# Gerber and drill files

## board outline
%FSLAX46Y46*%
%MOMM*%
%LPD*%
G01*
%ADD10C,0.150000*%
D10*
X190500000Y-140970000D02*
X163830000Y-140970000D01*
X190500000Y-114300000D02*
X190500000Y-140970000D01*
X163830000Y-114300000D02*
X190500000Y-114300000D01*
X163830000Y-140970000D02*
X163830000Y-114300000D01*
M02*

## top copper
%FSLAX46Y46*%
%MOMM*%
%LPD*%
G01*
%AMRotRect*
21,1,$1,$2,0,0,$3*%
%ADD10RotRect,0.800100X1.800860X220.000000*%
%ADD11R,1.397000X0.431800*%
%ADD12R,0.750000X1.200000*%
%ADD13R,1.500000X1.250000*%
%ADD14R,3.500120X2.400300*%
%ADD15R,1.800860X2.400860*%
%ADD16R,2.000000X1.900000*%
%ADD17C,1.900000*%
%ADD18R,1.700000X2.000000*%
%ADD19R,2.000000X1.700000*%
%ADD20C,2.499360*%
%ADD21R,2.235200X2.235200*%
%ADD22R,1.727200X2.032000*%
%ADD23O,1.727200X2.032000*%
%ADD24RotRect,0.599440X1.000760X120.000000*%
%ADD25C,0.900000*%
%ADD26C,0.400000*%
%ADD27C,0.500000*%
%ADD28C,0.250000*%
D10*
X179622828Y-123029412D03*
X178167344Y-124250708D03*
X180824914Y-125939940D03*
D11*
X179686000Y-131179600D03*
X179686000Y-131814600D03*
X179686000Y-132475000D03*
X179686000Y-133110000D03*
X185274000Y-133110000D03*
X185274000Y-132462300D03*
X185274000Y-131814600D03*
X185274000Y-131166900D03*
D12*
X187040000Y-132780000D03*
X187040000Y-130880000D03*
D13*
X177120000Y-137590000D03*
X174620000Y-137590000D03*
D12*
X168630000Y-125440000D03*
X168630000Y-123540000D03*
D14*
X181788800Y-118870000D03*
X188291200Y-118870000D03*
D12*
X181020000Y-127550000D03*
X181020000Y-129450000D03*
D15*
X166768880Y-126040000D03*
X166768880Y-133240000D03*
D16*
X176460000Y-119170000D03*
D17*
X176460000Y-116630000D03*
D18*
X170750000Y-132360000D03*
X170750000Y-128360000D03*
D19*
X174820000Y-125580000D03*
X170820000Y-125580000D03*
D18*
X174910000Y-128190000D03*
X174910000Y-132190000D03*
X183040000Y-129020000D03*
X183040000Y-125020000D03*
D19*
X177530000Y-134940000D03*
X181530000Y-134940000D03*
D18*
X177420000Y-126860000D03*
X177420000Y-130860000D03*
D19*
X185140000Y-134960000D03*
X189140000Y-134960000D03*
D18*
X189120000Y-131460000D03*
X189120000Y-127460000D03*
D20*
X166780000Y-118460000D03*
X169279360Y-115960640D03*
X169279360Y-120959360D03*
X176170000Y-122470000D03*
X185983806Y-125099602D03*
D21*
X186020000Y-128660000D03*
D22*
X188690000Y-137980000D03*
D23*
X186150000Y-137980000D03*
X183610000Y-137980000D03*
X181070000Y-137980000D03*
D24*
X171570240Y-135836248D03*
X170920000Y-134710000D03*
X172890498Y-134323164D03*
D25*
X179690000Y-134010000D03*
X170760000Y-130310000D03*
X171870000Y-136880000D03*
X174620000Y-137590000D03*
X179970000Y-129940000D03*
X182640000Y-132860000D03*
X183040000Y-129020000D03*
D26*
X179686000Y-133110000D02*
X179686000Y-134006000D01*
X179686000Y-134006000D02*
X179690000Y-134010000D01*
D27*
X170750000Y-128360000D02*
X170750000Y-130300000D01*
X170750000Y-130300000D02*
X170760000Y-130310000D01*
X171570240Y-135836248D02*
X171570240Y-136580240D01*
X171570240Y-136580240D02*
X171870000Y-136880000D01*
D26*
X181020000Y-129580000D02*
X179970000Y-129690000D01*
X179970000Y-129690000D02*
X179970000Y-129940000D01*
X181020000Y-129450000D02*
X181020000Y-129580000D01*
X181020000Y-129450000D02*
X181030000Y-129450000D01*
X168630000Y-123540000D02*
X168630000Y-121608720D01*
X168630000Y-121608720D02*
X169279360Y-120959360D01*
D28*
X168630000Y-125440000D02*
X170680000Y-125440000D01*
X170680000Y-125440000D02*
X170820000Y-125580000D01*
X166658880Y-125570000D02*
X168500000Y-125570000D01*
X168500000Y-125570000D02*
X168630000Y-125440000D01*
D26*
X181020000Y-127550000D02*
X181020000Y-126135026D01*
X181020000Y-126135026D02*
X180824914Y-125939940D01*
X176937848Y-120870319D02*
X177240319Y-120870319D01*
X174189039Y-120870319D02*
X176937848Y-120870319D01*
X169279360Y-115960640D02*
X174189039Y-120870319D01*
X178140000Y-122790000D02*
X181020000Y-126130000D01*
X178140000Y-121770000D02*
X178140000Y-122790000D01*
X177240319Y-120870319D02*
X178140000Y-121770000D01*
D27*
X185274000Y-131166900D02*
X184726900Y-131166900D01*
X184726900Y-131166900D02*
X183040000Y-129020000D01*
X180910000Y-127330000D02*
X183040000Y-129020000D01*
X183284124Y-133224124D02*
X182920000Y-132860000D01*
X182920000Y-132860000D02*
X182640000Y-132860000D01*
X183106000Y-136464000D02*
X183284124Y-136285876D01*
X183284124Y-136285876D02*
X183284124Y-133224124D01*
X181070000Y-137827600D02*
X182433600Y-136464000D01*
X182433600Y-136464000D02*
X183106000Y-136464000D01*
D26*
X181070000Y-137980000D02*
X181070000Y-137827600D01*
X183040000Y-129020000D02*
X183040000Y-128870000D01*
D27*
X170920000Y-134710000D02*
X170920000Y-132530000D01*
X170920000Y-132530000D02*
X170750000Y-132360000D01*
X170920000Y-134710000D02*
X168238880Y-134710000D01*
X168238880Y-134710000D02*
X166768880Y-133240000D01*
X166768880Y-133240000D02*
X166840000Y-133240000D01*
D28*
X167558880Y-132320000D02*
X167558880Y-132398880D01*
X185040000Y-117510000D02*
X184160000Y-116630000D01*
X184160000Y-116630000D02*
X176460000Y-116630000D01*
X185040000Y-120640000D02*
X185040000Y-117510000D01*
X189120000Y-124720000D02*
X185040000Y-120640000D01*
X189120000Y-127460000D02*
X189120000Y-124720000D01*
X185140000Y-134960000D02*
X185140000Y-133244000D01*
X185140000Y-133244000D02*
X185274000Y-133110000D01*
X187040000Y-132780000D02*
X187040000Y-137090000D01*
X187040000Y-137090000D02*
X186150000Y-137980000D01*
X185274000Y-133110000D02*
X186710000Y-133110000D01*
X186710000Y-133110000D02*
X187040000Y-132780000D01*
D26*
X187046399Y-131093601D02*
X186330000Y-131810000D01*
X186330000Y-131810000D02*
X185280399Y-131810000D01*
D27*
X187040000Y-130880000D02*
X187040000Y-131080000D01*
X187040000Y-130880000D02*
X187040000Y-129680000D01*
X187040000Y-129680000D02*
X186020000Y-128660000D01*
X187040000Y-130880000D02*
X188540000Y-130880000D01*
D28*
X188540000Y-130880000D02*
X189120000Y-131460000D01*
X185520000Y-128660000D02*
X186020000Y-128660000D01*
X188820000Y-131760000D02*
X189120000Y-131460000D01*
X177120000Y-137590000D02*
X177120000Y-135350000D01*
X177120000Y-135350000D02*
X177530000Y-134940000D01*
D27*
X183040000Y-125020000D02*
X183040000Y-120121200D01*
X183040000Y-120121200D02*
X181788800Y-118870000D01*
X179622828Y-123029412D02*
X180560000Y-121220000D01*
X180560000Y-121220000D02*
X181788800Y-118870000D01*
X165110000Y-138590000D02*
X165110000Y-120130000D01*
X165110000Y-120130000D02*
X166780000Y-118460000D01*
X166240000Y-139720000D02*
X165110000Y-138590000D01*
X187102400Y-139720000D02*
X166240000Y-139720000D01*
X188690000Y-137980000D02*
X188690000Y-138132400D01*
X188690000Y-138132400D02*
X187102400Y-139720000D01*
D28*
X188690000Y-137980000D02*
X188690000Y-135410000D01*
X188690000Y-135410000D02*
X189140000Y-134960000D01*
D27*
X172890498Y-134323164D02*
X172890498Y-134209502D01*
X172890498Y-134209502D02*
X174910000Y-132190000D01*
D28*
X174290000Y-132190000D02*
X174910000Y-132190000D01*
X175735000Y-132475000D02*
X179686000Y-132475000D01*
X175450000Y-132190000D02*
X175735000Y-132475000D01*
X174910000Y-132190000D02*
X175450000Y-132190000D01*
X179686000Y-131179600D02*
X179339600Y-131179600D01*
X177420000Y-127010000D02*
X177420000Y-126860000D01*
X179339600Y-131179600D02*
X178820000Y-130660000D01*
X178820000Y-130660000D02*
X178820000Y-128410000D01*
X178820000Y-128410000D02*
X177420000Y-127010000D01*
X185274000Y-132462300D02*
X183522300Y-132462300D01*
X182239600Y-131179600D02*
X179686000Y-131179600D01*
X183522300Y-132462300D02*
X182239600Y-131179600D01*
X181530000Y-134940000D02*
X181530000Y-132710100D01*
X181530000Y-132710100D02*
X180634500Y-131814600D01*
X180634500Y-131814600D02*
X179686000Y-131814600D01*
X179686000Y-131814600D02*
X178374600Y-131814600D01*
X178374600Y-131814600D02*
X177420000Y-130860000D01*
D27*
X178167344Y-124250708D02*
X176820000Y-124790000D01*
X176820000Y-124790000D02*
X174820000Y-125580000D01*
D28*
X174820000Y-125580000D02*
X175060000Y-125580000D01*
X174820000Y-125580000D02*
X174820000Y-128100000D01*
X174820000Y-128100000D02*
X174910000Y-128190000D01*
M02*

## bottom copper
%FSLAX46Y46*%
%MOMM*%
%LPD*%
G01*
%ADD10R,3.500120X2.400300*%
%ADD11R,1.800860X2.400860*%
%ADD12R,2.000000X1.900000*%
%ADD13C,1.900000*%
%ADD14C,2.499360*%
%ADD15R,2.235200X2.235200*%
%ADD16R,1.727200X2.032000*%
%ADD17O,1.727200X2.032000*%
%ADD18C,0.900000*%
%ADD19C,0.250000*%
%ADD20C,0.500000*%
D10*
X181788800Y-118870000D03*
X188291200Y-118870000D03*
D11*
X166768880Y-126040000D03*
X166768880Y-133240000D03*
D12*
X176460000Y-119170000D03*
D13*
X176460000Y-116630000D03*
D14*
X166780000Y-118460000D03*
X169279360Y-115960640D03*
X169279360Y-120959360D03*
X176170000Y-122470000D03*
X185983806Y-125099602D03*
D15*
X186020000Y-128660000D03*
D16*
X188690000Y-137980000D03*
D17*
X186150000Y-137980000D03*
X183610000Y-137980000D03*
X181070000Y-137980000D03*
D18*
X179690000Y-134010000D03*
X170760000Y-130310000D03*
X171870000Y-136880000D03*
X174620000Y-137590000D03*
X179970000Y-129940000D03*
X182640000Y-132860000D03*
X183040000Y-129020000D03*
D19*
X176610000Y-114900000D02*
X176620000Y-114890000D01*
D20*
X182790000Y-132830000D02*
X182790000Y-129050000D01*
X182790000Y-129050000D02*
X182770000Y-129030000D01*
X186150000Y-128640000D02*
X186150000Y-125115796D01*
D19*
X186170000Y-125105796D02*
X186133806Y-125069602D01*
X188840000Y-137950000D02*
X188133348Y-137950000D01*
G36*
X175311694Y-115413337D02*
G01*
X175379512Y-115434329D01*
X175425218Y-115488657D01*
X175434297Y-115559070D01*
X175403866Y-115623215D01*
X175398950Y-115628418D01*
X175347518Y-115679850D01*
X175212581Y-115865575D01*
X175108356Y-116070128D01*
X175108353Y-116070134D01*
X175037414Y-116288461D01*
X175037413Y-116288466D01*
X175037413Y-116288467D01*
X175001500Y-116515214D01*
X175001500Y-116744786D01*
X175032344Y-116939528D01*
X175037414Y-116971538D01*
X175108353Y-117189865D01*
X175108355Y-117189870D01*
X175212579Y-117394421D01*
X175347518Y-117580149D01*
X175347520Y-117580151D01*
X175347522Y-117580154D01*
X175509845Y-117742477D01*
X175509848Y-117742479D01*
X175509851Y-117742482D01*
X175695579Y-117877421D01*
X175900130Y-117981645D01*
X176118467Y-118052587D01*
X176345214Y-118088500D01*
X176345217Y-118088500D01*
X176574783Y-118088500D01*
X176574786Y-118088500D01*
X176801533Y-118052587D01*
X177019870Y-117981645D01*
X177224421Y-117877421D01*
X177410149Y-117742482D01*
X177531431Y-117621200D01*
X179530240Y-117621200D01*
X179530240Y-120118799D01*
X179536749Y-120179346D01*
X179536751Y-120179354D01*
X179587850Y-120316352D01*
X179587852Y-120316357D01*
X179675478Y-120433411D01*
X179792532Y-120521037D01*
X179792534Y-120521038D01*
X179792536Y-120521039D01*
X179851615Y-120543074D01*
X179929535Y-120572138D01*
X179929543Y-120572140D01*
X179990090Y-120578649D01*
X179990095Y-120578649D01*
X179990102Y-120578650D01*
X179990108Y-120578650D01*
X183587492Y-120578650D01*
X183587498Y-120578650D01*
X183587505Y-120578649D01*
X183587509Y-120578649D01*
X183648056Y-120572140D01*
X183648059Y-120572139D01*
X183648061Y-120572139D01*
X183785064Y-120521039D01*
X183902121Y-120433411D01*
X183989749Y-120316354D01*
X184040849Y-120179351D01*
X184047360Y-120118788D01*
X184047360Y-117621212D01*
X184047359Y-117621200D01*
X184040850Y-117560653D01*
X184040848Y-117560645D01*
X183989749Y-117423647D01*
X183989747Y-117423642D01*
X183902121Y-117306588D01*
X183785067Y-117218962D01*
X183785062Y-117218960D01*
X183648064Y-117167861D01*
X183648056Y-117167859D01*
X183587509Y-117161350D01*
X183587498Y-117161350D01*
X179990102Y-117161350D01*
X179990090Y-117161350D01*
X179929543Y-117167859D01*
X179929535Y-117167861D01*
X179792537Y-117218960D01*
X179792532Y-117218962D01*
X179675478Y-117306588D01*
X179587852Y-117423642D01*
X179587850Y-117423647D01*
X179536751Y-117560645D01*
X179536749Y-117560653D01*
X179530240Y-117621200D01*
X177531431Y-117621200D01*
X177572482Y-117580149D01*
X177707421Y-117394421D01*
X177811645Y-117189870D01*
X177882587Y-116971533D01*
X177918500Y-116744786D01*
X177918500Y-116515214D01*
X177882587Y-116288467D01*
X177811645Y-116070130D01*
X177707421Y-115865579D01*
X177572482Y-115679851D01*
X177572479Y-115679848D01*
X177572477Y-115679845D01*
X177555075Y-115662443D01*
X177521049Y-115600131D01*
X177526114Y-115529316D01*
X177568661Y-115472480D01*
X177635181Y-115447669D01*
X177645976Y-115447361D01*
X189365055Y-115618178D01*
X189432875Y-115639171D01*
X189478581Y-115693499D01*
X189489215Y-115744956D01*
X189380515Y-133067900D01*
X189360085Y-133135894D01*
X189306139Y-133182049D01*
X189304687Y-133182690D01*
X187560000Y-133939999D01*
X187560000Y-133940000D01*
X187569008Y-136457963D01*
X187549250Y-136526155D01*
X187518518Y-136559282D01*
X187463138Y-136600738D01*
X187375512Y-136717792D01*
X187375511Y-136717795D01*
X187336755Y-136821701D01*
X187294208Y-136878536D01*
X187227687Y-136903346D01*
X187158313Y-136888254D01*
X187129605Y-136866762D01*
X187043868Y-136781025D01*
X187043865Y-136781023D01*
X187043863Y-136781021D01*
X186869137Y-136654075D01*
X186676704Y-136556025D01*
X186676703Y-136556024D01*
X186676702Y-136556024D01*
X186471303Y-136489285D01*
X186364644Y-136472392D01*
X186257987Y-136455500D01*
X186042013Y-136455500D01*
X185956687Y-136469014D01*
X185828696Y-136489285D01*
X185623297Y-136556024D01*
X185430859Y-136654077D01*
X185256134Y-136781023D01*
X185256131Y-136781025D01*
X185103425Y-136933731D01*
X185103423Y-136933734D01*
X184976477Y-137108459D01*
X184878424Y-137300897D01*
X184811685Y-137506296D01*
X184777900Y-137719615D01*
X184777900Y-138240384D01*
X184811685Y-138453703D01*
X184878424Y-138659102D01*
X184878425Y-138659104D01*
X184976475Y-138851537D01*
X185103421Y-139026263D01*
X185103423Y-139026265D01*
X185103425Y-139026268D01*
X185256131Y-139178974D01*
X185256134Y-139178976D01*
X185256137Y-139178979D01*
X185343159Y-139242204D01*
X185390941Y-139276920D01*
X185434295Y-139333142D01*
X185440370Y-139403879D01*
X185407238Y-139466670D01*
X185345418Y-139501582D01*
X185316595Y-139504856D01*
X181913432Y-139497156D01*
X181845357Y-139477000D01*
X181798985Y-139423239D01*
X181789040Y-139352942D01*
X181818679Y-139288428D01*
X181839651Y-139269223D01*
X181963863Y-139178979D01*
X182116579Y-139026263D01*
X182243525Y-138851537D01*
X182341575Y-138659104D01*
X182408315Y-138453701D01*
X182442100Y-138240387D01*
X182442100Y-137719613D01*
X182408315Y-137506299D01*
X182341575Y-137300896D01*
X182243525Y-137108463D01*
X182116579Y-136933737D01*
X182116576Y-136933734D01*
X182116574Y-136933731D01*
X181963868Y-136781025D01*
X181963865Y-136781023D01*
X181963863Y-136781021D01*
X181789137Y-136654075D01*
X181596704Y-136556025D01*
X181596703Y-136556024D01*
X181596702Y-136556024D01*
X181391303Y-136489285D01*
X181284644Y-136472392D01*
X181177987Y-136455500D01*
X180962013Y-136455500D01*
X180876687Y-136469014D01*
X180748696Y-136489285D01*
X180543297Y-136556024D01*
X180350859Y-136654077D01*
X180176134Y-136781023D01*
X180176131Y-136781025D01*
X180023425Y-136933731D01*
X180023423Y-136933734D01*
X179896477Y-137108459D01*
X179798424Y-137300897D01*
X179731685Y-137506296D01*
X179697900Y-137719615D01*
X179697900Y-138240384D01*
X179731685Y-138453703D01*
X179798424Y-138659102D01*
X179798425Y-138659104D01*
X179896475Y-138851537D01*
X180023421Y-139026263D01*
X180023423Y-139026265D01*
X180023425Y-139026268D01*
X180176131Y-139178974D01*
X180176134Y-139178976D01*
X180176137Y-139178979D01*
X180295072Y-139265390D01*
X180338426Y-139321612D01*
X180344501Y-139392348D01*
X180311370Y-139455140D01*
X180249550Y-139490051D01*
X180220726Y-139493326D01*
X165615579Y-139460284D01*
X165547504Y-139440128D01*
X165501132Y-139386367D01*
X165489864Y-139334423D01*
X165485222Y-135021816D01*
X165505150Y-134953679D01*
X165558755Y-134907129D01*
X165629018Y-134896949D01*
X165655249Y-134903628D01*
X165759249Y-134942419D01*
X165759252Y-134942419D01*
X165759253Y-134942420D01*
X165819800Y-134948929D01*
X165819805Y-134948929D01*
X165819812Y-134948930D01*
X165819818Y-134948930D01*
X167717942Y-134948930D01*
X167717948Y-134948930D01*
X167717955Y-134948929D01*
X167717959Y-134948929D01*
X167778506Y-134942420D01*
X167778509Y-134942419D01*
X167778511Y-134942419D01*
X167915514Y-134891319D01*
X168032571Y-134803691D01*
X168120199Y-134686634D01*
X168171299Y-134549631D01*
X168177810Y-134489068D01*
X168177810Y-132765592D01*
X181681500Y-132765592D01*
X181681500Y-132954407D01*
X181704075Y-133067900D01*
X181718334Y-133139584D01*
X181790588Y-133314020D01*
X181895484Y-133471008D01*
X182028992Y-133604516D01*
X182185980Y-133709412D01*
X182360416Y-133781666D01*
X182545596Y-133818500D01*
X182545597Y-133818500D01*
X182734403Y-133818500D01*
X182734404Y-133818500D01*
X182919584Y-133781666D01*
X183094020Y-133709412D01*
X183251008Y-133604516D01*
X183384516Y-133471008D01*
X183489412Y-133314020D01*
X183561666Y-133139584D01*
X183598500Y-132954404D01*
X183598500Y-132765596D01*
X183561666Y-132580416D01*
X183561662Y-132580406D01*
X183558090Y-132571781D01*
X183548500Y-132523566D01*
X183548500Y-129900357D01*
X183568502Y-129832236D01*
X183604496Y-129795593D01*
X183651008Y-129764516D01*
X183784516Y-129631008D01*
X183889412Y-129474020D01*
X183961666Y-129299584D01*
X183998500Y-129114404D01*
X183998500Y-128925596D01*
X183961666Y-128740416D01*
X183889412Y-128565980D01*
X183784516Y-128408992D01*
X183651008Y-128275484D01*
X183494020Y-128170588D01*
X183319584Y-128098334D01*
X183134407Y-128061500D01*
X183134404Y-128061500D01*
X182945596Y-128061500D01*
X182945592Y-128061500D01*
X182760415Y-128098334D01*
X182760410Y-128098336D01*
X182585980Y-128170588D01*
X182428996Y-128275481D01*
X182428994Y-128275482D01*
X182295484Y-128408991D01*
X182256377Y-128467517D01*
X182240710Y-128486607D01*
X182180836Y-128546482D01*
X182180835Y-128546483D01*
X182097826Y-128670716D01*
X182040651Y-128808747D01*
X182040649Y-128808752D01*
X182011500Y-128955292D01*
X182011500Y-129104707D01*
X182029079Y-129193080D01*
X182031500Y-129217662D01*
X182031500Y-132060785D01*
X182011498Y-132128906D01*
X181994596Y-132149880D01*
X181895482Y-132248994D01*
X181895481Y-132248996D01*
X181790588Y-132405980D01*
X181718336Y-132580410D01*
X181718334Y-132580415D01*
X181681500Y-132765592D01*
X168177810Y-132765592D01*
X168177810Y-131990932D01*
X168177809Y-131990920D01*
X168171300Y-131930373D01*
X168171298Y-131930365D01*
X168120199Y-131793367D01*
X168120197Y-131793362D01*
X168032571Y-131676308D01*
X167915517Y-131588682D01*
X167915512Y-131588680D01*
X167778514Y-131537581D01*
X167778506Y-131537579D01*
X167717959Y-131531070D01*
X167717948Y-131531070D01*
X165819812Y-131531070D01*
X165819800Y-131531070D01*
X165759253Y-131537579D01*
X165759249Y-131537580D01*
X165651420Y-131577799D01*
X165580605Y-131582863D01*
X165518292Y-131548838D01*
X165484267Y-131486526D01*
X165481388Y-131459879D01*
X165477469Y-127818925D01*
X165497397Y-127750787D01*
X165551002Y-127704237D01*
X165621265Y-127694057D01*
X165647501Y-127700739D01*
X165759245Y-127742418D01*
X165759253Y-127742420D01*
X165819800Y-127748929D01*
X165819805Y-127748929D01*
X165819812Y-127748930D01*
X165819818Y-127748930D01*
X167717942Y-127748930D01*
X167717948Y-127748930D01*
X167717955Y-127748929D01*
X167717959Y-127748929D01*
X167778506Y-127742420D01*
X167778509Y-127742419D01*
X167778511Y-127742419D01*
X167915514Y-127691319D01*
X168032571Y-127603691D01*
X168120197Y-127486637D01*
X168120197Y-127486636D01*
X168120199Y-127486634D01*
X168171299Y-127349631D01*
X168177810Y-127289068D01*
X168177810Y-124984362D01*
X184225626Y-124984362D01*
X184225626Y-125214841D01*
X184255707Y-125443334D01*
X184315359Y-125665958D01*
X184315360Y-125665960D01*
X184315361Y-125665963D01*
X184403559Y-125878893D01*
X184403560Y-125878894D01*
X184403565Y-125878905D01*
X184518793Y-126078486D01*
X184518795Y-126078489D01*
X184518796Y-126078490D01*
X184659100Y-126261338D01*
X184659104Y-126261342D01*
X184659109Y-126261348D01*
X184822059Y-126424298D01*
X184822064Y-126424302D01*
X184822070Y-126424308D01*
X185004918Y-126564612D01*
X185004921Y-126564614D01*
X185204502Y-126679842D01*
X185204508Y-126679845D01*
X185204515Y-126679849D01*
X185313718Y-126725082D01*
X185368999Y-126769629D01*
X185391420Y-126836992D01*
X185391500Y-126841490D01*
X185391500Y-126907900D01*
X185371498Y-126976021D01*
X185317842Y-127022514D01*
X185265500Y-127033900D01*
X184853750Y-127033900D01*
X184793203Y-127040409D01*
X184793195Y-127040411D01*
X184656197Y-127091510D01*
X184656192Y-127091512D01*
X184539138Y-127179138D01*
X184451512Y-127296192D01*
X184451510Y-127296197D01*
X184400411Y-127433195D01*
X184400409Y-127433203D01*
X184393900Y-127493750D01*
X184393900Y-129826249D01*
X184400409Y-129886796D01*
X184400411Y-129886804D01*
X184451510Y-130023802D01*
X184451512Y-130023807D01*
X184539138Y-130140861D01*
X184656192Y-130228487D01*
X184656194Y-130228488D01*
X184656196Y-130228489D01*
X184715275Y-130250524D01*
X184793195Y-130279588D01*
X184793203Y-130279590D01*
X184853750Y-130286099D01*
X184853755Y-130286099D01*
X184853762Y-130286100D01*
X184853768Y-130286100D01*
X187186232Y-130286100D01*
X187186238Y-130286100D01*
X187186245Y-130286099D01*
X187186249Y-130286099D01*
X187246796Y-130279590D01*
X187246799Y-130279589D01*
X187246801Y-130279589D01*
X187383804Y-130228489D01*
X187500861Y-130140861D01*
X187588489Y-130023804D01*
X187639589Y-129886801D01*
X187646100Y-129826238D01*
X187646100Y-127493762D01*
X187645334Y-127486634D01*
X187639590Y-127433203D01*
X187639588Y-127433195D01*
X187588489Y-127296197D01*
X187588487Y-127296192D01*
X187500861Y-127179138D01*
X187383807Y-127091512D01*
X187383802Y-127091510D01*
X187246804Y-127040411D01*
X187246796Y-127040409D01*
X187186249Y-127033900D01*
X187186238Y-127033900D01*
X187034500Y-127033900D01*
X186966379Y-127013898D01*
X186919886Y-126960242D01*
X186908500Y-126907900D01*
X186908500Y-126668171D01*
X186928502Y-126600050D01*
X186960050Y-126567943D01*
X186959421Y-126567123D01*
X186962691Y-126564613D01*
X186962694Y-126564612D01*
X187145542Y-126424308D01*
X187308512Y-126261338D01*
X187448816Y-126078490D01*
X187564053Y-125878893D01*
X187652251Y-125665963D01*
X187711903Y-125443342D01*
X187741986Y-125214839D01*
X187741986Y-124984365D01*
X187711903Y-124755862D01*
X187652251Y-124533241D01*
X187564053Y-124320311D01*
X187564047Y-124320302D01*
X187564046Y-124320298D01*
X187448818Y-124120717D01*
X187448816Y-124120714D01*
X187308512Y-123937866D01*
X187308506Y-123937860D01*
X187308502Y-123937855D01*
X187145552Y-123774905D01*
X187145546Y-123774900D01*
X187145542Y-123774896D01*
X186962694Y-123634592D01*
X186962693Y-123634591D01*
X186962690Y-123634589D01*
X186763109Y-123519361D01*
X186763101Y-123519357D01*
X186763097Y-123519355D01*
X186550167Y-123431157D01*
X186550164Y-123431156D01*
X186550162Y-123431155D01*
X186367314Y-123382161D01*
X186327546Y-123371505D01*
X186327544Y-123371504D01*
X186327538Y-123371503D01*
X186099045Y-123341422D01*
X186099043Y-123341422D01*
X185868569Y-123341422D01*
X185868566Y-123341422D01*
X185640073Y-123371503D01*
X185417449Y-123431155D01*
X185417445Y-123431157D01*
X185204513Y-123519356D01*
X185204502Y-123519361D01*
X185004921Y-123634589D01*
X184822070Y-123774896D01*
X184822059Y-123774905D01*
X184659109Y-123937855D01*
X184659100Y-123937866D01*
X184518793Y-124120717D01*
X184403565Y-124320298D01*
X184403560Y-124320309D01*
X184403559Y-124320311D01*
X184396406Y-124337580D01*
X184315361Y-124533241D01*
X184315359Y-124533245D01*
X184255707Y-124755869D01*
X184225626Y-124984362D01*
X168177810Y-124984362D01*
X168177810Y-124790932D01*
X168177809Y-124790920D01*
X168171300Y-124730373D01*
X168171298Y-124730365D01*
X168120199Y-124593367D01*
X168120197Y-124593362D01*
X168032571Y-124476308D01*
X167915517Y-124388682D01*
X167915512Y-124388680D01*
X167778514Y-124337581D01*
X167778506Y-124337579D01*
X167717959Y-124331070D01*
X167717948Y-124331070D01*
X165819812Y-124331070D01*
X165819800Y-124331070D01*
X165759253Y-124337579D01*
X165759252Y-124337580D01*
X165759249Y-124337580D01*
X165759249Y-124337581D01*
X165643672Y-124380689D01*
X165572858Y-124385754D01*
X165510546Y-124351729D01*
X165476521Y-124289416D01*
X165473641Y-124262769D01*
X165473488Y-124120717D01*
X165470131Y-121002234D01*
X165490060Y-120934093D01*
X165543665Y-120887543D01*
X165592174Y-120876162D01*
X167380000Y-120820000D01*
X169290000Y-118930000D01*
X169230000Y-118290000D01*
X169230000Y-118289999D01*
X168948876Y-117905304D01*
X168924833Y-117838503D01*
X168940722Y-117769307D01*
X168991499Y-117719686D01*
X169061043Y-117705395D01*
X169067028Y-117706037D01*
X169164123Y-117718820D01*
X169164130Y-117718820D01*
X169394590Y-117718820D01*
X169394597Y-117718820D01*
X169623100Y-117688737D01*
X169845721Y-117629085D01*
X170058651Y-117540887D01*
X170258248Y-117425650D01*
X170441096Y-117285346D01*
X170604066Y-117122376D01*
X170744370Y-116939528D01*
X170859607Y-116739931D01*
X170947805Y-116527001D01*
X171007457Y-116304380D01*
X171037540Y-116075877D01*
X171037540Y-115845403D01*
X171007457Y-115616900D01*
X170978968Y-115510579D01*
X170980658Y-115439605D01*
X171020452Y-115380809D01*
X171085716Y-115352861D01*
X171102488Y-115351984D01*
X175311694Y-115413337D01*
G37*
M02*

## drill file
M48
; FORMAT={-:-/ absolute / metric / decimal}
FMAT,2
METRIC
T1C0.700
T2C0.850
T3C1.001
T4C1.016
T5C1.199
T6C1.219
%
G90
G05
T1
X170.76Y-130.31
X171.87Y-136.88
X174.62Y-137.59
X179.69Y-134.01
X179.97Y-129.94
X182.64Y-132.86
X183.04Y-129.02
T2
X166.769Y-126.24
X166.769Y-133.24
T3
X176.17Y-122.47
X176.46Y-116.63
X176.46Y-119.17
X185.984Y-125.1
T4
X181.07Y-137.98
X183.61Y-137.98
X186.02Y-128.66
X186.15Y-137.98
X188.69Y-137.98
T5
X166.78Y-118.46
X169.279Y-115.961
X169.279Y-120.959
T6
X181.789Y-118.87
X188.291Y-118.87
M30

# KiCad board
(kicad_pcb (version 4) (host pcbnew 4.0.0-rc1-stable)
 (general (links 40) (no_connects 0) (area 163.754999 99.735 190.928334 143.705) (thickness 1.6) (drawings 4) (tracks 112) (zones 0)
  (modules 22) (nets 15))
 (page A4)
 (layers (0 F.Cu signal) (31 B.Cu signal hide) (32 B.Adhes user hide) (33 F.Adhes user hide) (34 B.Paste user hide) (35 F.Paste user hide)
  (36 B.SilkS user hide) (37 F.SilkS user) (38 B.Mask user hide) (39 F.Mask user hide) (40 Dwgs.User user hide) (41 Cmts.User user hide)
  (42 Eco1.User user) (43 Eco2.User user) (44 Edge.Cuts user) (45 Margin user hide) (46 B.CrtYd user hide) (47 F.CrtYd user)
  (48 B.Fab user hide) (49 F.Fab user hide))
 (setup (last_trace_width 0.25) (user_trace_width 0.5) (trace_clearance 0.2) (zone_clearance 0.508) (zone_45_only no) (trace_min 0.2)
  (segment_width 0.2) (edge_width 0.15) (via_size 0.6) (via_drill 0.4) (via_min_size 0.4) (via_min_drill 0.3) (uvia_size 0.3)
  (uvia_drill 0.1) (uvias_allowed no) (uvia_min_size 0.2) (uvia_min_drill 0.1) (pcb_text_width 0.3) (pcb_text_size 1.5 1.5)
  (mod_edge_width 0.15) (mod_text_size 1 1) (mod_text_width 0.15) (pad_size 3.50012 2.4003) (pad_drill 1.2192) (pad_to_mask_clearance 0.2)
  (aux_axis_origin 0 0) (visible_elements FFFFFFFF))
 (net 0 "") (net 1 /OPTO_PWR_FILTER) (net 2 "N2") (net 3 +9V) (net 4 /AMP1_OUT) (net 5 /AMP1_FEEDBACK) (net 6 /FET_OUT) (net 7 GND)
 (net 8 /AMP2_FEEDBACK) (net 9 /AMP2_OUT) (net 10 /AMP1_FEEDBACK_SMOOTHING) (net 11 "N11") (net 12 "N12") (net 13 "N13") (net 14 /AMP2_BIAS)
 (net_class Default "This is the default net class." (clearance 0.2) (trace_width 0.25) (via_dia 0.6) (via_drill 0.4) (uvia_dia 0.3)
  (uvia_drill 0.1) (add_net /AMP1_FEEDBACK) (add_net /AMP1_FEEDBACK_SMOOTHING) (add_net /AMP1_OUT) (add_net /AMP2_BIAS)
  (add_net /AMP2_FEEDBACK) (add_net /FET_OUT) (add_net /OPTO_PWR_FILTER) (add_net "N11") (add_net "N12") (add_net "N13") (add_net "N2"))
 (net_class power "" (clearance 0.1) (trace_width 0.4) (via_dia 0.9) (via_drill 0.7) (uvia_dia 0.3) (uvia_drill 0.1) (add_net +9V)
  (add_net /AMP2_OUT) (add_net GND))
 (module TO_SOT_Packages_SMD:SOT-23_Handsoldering (layer F.Cu) (at 179.86 124.79 220)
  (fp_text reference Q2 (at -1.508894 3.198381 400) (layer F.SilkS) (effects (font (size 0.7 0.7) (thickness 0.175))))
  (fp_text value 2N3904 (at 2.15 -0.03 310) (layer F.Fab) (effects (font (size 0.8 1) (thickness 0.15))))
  (pad 1 smd rect (at -0.95 1.50114 220) (size 0.8001 1.80086) (layers F.Cu F.Paste F.Mask) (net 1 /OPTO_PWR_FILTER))
  (pad 2 smd rect (at 0.95 1.50114 220) (size 0.8001 1.80086) (layers F.Cu F.Paste F.Mask) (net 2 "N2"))
  (pad 3 smd rect (at 0 -1.50114 220) (size 0.8001 1.80086) (layers F.Cu F.Paste F.Mask) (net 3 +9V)))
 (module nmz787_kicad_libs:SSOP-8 (layer F.Cu) (at 182.48 133.11 270)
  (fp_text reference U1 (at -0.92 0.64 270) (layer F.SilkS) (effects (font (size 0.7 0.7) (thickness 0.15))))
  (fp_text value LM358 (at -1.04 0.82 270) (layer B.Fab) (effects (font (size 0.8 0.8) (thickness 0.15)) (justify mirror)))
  (pad 1 smd rect (at -1.9304 2.794 270) (size 0.4318 1.397) (layers F.Cu F.Paste F.Mask) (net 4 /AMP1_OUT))
  (pad 2 smd rect (at -1.2954 2.794 270) (size 0.4318 1.397) (layers F.Cu F.Paste F.Mask) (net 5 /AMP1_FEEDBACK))
  (pad 3 smd rect (at -0.635 2.794 270) (size 0.4318 1.397) (layers F.Cu F.Paste F.Mask) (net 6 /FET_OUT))
  (pad 4 smd rect (at 0 2.794 270) (size 0.4318 1.397) (layers F.Cu F.Paste F.Mask) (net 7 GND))
  (pad 5 smd rect (at 0 -2.794 270) (size 0.4318 1.397) (layers F.Cu F.Paste F.Mask) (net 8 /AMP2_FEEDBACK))
  (pad 6 smd rect (at -0.6477 -2.794 270) (size 0.4318 1.397) (layers F.Cu F.Paste F.Mask) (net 4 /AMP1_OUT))
  (pad 7 smd rect (at -1.2954 -2.794 270) (size 0.4318 1.397) (layers F.Cu F.Paste F.Mask) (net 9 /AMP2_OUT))
  (pad 8 smd rect (at -1.9431 -2.794 270) (size 0.4318 1.397) (layers F.Cu F.Paste F.Mask) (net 3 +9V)))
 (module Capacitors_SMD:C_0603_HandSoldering (layer F.Cu) (at 187.04 131.83 90)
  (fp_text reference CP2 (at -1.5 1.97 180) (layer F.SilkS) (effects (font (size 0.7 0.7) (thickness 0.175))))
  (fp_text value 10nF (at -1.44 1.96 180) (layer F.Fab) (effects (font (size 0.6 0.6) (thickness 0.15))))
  (pad 1 smd rect (at -0.95 0 90) (size 1.2 0.75) (layers F.Cu F.Paste F.Mask) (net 8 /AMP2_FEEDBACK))
  (pad 2 smd rect (at 0.95 0 90) (size 1.2 0.75) (layers F.Cu F.Paste F.Mask) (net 9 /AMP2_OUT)))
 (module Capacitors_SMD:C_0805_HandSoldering (layer F.Cu) (at 175.87 137.59 180)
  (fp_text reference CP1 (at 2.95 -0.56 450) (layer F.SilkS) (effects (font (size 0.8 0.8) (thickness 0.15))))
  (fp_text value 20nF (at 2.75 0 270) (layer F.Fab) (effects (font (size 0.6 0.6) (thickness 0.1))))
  (pad 1 smd rect (at -1.25 0 180) (size 1.5 1.25) (layers F.Cu F.Paste F.Mask) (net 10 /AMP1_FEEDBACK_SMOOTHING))
  (pad 2 smd rect (at 1.25 0 180) (size 1.5 1.25) (layers F.Cu F.Paste F.Mask) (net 7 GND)))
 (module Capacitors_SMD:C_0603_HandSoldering (layer F.Cu) (at 168.63 124.49 90)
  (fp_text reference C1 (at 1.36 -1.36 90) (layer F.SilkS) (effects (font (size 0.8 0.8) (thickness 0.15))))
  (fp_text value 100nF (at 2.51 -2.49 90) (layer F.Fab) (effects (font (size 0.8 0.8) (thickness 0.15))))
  (pad 1 smd rect (at -0.95 0 90) (size 1.2 0.75) (layers F.Cu F.Paste F.Mask) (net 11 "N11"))
  (pad 2 smd rect (at 0.95 0 90) (size 1.2 0.75) (layers F.Cu F.Paste F.Mask) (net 7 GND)))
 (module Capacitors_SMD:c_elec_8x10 (layer F.Cu) (at 185.04 118.87 180)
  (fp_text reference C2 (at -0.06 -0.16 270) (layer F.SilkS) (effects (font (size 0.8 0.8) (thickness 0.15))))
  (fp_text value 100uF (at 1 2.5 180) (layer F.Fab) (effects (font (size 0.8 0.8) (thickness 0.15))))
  (pad 1 thru_hole rect (at 3.2512 0 180) (size 3.50012 2.4003) (drill 1.2192) (layers *.Cu *.Mask F.SilkS) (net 1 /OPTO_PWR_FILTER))
  (pad 2 thru_hole rect (at -3.2512 0 180) (size 3.50012 2.4003) (drill 1.2192) (layers *.Cu *.Mask F.SilkS) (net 7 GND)))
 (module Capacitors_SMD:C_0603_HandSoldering (layer F.Cu) (at 181.02 128.5 270)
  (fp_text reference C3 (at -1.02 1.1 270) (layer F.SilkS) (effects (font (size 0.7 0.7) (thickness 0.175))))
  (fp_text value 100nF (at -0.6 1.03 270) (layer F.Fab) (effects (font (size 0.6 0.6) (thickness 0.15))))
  (pad 1 smd rect (at -0.95 0 270) (size 1.2 0.75) (layers F.Cu F.Paste F.Mask) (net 3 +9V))
  (pad 2 smd rect (at 0.95 0 270) (size 1.2 0.75) (layers F.Cu F.Paste F.Mask) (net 7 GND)))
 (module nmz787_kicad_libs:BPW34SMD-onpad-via (layer F.Cu) (at 166.84 129.74 270)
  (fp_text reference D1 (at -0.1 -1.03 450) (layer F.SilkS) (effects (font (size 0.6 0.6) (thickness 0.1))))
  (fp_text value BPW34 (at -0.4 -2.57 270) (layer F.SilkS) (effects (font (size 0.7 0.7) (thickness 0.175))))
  (pad 1 thru_hole rect (at -3.5 0.07112 270) (size 2.40086 1.80086) (drill 0.85 (offset -0.2 0)) (layers *.Cu *.Mask F.SilkS)
   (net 11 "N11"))
  (pad 2 thru_hole rect (at 3.5 0.07112 270) (size 2.40086 1.80086) (drill 0.85) (layers *.Cu *.Mask F.SilkS) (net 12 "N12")))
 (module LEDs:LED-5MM (layer F.Cu) (at 176.46 119.17 90)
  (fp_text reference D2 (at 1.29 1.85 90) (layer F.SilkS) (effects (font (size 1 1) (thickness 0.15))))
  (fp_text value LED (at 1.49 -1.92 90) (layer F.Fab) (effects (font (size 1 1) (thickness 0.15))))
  (pad 1 thru_hole rect (at 0 0 180) (size 2 1.9) (drill 1.00076) (layers *.Cu *.Mask F.SilkS) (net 7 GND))
  (pad 2 thru_hole circle (at 2.54 0 90) (size 1.9 1.9) (drill 1.00076) (layers *.Cu *.Mask F.SilkS) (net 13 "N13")))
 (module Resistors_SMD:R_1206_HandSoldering (layer F.Cu) (at 170.75 130.36 90)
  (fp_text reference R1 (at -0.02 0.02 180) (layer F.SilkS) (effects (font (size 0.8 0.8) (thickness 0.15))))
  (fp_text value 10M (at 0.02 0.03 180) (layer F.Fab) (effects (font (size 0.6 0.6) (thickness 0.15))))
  (pad 1 smd rect (at -2 0 90) (size 2 1.7) (layers F.Cu F.Paste F.Mask) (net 12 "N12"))
  (pad 2 smd rect (at 2 0 90) (size 2 1.7) (layers F.Cu F.Paste F.Mask) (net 7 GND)))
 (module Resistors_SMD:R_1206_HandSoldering (layer F.Cu) (at 172.82 125.58 180)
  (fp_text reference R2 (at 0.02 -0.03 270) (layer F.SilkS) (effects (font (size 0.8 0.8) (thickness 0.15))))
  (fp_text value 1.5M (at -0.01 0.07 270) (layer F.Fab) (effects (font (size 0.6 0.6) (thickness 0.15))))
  (pad 1 smd rect (at -2 0 180) (size 2 1.7) (layers F.Cu F.Paste F.Mask) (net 2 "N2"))
  (pad 2 smd rect (at 2 0 180) (size 2 1.7) (layers F.Cu F.Paste F.Mask) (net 11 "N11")))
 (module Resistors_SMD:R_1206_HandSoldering (layer F.Cu) (at 174.91 130.19 270)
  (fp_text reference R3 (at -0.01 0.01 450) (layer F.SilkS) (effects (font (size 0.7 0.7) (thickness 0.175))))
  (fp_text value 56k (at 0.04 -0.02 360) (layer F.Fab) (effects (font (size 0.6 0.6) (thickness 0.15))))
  (pad 1 smd rect (at -2 0 270) (size 2 1.7) (layers F.Cu F.Paste F.Mask) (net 2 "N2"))
  (pad 2 smd rect (at 2 0 270) (size 2 1.7) (layers F.Cu F.Paste F.Mask) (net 6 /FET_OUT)))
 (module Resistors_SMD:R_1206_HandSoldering (layer F.Cu) (at 183.04 127.02 90)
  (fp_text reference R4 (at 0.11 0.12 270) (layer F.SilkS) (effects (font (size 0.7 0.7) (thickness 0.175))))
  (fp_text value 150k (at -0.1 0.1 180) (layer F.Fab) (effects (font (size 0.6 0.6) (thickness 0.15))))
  (pad 1 smd rect (at -2 0 90) (size 2 1.7) (layers F.Cu F.Paste F.Mask) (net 3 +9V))
  (pad 2 smd rect (at 2 0 90) (size 2 1.7) (layers F.Cu F.Paste F.Mask) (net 1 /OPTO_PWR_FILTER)))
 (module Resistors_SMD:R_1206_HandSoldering (layer F.Cu) (at 179.53 134.94)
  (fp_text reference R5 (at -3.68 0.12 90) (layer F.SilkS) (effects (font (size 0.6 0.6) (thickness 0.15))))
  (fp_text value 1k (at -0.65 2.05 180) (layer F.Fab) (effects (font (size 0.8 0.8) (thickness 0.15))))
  (pad 1 smd rect (at -2 0) (size 2 1.7) (layers F.Cu F.Paste F.Mask) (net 10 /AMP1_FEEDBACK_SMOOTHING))
  (pad 2 smd rect (at 2 0) (size 2 1.7) (layers F.Cu F.Paste F.Mask) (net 5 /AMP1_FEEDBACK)))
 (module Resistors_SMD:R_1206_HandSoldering (layer F.Cu) (at 177.42 128.86 270)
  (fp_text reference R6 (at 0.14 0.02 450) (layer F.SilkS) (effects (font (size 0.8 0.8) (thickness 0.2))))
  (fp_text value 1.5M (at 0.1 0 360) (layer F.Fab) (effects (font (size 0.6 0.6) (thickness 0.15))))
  (pad 1 smd rect (at -2 0 270) (size 2 1.7) (layers F.Cu F.Paste F.Mask) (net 4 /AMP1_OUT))
  (pad 2 smd rect (at 2 0 270) (size 2 1.7) (layers F.Cu F.Paste F.Mask) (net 5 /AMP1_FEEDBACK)))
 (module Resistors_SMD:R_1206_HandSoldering (layer F.Cu) (at 187.14 134.96)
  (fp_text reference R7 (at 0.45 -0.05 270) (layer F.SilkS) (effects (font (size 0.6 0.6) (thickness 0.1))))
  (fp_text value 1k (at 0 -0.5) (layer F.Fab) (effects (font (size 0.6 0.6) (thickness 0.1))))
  (pad 1 smd rect (at -2 0) (size 2 1.7) (layers F.Cu F.Paste F.Mask) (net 8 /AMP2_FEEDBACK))
  (pad 2 smd rect (at 2 0) (size 2 1.7) (layers F.Cu F.Paste F.Mask) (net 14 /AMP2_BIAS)))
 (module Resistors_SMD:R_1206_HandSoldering (layer F.Cu) (at 189.12 129.46 90)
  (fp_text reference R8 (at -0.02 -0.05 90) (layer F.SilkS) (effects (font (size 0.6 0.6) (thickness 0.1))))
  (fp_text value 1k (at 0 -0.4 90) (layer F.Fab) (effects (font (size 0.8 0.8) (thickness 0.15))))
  (pad 1 smd rect (at -2 0 90) (size 2 1.7) (layers F.Cu F.Paste F.Mask) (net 9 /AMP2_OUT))
  (pad 2 smd rect (at 2 0 90) (size 2 1.7) (layers F.Cu F.Paste F.Mask) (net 13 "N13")))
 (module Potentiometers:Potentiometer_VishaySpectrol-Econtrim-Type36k (layer F.Cu) (at 169.27936 120.95936 90)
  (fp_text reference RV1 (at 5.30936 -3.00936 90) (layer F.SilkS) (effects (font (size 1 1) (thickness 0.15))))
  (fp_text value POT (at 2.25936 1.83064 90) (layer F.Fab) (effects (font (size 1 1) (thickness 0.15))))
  (pad 2 thru_hole circle (at 2.49936 -2.49936 90) (size 2.49936 2.49936) (drill 1.19888) (layers *.Cu *.Mask F.SilkS) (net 14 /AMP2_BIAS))
  (pad 3 thru_hole circle (at 4.99872 0 90) (size 2.49936 2.49936) (drill 1.19888) (layers *.Cu *.Mask F.SilkS) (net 3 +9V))
  (pad 1 thru_hole circle (at 0 0 90) (size 2.49936 2.49936) (drill 1.19888) (layers *.Cu *.Mask F.SilkS) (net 7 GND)))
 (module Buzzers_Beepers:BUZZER (layer B.Cu) (at 181.076903 123.784801 165)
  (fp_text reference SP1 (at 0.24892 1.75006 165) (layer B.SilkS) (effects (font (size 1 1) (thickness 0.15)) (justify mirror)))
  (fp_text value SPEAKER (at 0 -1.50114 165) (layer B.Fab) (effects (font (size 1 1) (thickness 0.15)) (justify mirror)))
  (pad 2 thru_hole circle (at 5.08 0 165) (size 2.49936 2.49936) (drill 1.00076) (layers *.Cu *.Mask B.SilkS) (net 7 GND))
  (pad 1 thru_hole circle (at -5.08 0 165) (size 2.49936 2.49936) (drill 1.00076) (layers *.Cu *.Mask B.SilkS) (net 9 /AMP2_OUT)))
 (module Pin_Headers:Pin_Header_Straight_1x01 (layer F.Cu) (at 186.02 128.66)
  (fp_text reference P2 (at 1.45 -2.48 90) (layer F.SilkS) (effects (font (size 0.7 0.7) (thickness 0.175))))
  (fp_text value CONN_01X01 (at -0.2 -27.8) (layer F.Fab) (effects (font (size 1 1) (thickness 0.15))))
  (pad 1 thru_hole rect (at 0 0) (size 2.2352 2.2352) (drill 1.016) (layers *.Cu *.Mask F.SilkS) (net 9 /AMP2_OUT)))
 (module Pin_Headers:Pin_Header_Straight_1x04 (layer F.Cu) (at 188.69 137.98 270)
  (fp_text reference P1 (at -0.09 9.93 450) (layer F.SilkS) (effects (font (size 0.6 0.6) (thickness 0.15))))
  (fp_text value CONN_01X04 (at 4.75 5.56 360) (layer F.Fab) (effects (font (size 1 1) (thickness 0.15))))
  (pad 1 thru_hole rect (at 0 0 270) (size 2.032 1.7272) (drill 1.016) (layers *.Cu *.Mask F.SilkS) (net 14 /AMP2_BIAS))
  (pad 2 thru_hole oval (at 0 2.54 270) (size 2.032 1.7272) (drill 1.016) (layers *.Cu *.Mask F.SilkS) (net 8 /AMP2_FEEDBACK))
  (pad 3 thru_hole oval (at 0 5.08 270) (size 2.032 1.7272) (drill 1.016) (layers *.Cu *.Mask F.SilkS) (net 7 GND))
  (pad 4 thru_hole oval (at 0 7.62 270) (size 2.032 1.7272) (drill 1.016) (layers *.Cu *.Mask F.SilkS) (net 3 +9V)))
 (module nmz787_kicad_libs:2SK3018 (layer F.Cu) (at 172.067809 134.798144 120)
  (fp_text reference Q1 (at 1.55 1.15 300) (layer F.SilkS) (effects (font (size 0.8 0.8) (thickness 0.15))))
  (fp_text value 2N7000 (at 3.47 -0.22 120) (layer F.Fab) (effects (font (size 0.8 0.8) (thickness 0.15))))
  (pad 1 smd rect (at -0.65024 -0.94996 120) (size 0.59944 1.00076) (layers F.Cu F.Paste F.Mask) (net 7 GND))
  (pad 2 smd rect (at 0.65024 -0.94996 120) (size 0.59944 1.00076) (layers F.Cu F.Paste F.Mask) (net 12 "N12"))
  (pad 3 smd rect (at 0 0.94996 120) (size 0.59944 1.00076) (layers F.Cu F.Paste F.Mask) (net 6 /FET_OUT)))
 (gr_line (start 190.5 140.97) (end 163.83 140.97) (layer Edge.Cuts) (width 0.15))
 (gr_line (start 190.5 114.3) (end 190.5 140.97) (layer Edge.Cuts) (width 0.15))
 (gr_line (start 163.83 114.3) (end 190.5 114.3) (layer Edge.Cuts) (width 0.15))
 (gr_line (start 163.83 140.97) (end 163.83 114.3) (layer Edge.Cuts) (width 0.15))
 (segment (start 176.61 114.9) (end 176.62 114.89) (width 0.25) (layer B.Cu) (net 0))
 (segment (start 179.686 133.11) (end 179.686 134.006) (width 0.4) (layer F.Cu) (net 7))
 (segment (start 179.686 134.006) (end 179.69 134.01) (width 0.4) (layer F.Cu) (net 7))
 (via (at 179.69 134.01) (size 0.9) (drill 0.7) (layers F.Cu B.Cu) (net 7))
 (segment (start 170.75 128.36) (end 170.75 130.3) (width 0.5) (layer F.Cu) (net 7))
 (segment (start 170.75 130.3) (end 170.76 130.31) (width 0.5) (layer F.Cu) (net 7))
 (via (at 170.76 130.31) (size 0.9) (drill 0.7) (layers F.Cu B.Cu) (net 7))
 (segment (start 171.57024 135.836248) (end 171.57024 136.58024) (width 0.5) (layer F.Cu) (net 7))
 (segment (start 171.57024 136.58024) (end 171.87 136.88) (width 0.5) (layer F.Cu) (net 7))
 (via (at 171.87 136.88) (size 0.9) (drill 0.7) (layers F.Cu B.Cu) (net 7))
 (via (at 174.62 137.59) (size 0.9) (drill 0.7) (layers F.Cu B.Cu) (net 7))
 (segment (start 181.02 129.58) (end 179.97 129.69) (width 0.4) (layer F.Cu) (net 7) (status 10))
 (segment (start 179.97 129.69) (end 179.97 129.94) (width 0.4) (layer F.Cu) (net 7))
 (via (at 179.97 129.94) (size 0.9) (drill 0.7) (layers F.Cu B.Cu) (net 7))
 (segment (start 181.02 129.45) (end 181.02 129.58) (width 0.4) (layer F.Cu) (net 7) (status 30))
 (segment (start 181.02 129.45) (end 181.03 129.45) (width 0.4) (layer F.Cu) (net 7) (status 30))
 (segment (start 168.63 123.54) (end 168.63 121.60872) (width 0.4) (layer F.Cu) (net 7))
 (segment (start 168.63 121.60872) (end 169.27936 120.95936) (width 0.4) (layer F.Cu) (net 7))
 (segment (start 168.63 125.44) (end 170.68 125.44) (width 0.25) (layer F.Cu) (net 11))
 (segment (start 170.68 125.44) (end 170.82 125.58) (width 0.25) (layer F.Cu) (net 11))
 (segment (start 166.65888 125.57) (end 168.5 125.57) (width 0.25) (layer F.Cu) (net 11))
 (segment (start 168.5 125.57) (end 168.63 125.44) (width 0.25) (layer F.Cu) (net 11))
 (segment (start 181.02 127.55) (end 181.02 126.135026) (width 0.4) (layer F.Cu) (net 3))
 (segment (start 181.02 126.135026) (end 180.824914 125.93994) (width 0.4) (layer F.Cu) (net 3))
 (segment (start 176.937848 120.870319) (end 177.240319 120.870319) (width 0.4) (layer F.Cu) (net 3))
 (segment (start 174.189039 120.870319) (end 176.937848 120.870319) (width 0.4) (layer F.Cu) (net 3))
 (segment (start 169.27936 115.96064) (end 174.189039 120.870319) (width 0.4) (layer F.Cu) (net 3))
 (segment (start 178.14 122.79) (end 181.02 126.13) (width 0.4) (layer F.Cu) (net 3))
 (segment (start 178.14 121.77) (end 178.14 122.79) (width 0.4) (layer F.Cu) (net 3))
 (segment (start 177.240319 120.870319) (end 178.14 121.77) (width 0.4) (layer F.Cu) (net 3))
 (segment (start 185.274 131.1669) (end 184.7269 131.1669) (width 0.5) (layer F.Cu) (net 3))
 (segment (start 184.7269 131.1669) (end 183.04 129.02) (width 0.5) (layer F.Cu) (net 3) (status 20))
 (segment (start 180.91 127.33) (end 183.04 129.02) (width 0.5) (layer F.Cu) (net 3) (status 10))
 (segment (start 182.79 132.83) (end 182.79 129.05) (width 0.5) (layer B.Cu) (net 3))
 (segment (start 182.79 129.05) (end 182.77 129.03) (width 0.5) (layer B.Cu) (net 3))
 (segment (start 183.284124 133.224124) (end 182.92 132.86) (width 0.5) (layer F.Cu) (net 3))
 (segment (start 182.92 132.86) (end 182.64 132.86) (width 0.5) (layer F.Cu) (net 3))
 (via (at 182.64 132.86) (size 0.9) (drill 0.7) (layers F.Cu B.Cu) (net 3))
 (segment (start 183.106 136.464) (end 183.284124 136.285876) (width 0.5) (layer F.Cu) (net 3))
 (segment (start 183.284124 136.285876) (end 183.284124 133.224124) (width 0.5) (layer F.Cu) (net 3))
 (segment (start 181.07 137.8276) (end 182.4336 136.464) (width 0.5) (layer F.Cu) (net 3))
 (segment (start 182.4336 136.464) (end 183.106 136.464) (width 0.5) (layer F.Cu) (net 3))
 (segment (start 181.07 137.98) (end 181.07 137.8276) (width 0.4) (layer F.Cu) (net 3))
 (via (at 183.04 129.02) (size 0.9) (drill 0.7) (layers F.Cu B.Cu) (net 3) (status 30))
 (segment (start 183.04 129.02) (end 183.04 128.87) (width 0.4) (layer F.Cu) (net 3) (status 30))
 (segment (start 170.92 134.71) (end 170.92 132.53) (width 0.5) (layer F.Cu) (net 12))
 (segment (start 170.92 132.53) (end 170.75 132.36) (width 0.5) (layer F.Cu) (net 12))
 (segment (start 170.92 134.71) (end 168.23888 134.71) (width 0.5) (layer F.Cu) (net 12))
 (segment (start 168.23888 134.71) (end 166.76888 133.24) (width 0.5) (layer F.Cu) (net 12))
 (segment (start 166.76888 133.24) (end 166.84 133.24) (width 0.5) (layer F.Cu) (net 12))
 (segment (start 167.55888 132.32) (end 167.55888 132.39888) (width 0.25) (layer F.Cu) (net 12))
 (segment (start 185.04 117.51) (end 184.16 116.63) (width 0.25) (layer F.Cu) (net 13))
 (segment (start 184.16 116.63) (end 176.46 116.63) (width 0.25) (layer F.Cu) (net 13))
 (segment (start 185.04 120.64) (end 185.04 117.51) (width 0.25) (layer F.Cu) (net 13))
 (segment (start 189.12 124.72) (end 185.04 120.64) (width 0.25) (layer F.Cu) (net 13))
 (segment (start 189.12 127.46) (end 189.12 124.72) (width 0.25) (layer F.Cu) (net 13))
 (segment (start 185.14 134.96) (end 185.14 133.244) (width 0.25) (layer F.Cu) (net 8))
 (segment (start 185.14 133.244) (end 185.274 133.11) (width 0.25) (layer F.Cu) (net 8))
 (segment (start 187.04 132.78) (end 187.04 137.09) (width 0.25) (layer F.Cu) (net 8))
 (segment (start 187.04 137.09) (end 186.15 137.98) (width 0.25) (layer F.Cu) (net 8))
 (segment (start 185.274 133.11) (end 186.71 133.11) (width 0.25) (layer F.Cu) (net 8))
 (segment (start 186.71 133.11) (end 187.04 132.78) (width 0.25) (layer F.Cu) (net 8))
 (segment (start 187.046399 131.093601) (end 186.33 131.81) (width 0.4) (layer F.Cu) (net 9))
 (segment (start 186.33 131.81) (end 185.280399 131.81) (width 0.4) (layer F.Cu) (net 9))
 (segment (start 187.04 130.88) (end 187.04 131.08) (width 0.5) (layer F.Cu) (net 9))
 (segment (start 187.04 130.88) (end 187.04 129.68) (width 0.5) (layer F.Cu) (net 9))
 (segment (start 187.04 129.68) (end 186.02 128.66) (width 0.5) (layer F.Cu) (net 9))
 (segment (start 187.04 130.88) (end 188.54 130.88) (width 0.5) (layer F.Cu) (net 9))
 (segment (start 188.54 130.88) (end 189.12 131.46) (width 0.25) (layer F.Cu) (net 9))
 (segment (start 186.15 128.64) (end 186.15 125.115796) (width 0.5) (layer B.Cu) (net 9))
 (segment (start 186.17 125.105796) (end 186.133806 125.069602) (width 0.25) (layer B.Cu) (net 9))
 (segment (start 185.52 128.66) (end 186.02 128.66) (width 0.25) (layer F.Cu) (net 9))
 (segment (start 188.82 131.76) (end 189.12 131.46) (width 0.25) (layer F.Cu) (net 9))
 (segment (start 177.12 137.59) (end 177.12 135.35) (width 0.25) (layer F.Cu) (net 10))
 (segment (start 177.12 135.35) (end 177.53 134.94) (width 0.25) (layer F.Cu) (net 10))
 (segment (start 183.04 125.02) (end 183.04 120.1212) (width 0.5) (layer F.Cu) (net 1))
 (segment (start 183.04 120.1212) (end 181.7888 118.87) (width 0.5) (layer F.Cu) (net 1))
 (segment (start 179.622828 123.029412) (end 180.56 121.22) (width 0.5) (layer F.Cu) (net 1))
 (segment (start 180.56 121.22) (end 181.7888 118.87) (width 0.5) (layer F.Cu) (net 1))
 (segment (start 165.11 138.59) (end 165.11 120.13) (width 0.5) (layer F.Cu) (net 14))
 (segment (start 165.11 120.13) (end 166.78 118.46) (width 0.5) (layer F.Cu) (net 14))
 (segment (start 166.24 139.72) (end 165.11 138.59) (width 0.5) (layer F.Cu) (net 14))
 (segment (start 187.1024 139.72) (end 166.24 139.72) (width 0.5) (layer F.Cu) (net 14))
 (segment (start 188.69 137.98) (end 188.69 138.1324) (width 0.5) (layer F.Cu) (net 14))
 (segment (start 188.69 138.1324) (end 187.1024 139.72) (width 0.5) (layer F.Cu) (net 14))
 (segment (start 188.84 137.95) (end 188.133348 137.95) (width 0.25) (layer B.Cu) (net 14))
 (segment (start 188.69 137.98) (end 188.69 135.41) (width 0.25) (layer F.Cu) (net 14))
 (segment (start 188.69 135.41) (end 189.14 134.96) (width 0.25) (layer F.Cu) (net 14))
 (segment (start 172.890498 134.323164) (end 172.890498 134.209502) (width 0.5) (layer F.Cu) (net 6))
 (segment (start 172.890498 134.209502) (end 174.91 132.19) (width 0.5) (layer F.Cu) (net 6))
 (segment (start 174.29 132.19) (end 174.91 132.19) (width 0.25) (layer F.Cu) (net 6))
 (segment (start 175.735 132.475) (end 179.686 132.475) (width 0.25) (layer F.Cu) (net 6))
 (segment (start 175.45 132.19) (end 175.735 132.475) (width 0.25) (layer F.Cu) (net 6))
 (segment (start 174.91 132.19) (end 175.45 132.19) (width 0.25) (layer F.Cu) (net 6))
 (segment (start 179.686 131.1796) (end 179.3396 131.1796) (width 0.25) (layer F.Cu) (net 4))
 (segment (start 177.42 127.01) (end 177.42 126.86) (width 0.25) (layer F.Cu) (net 4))
 (segment (start 179.3396 131.1796) (end 178.82 130.66) (width 0.25) (layer F.Cu) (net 4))
 (segment (start 178.82 130.66) (end 178.82 128.41) (width 0.25) (layer F.Cu) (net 4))
 (segment (start 178.82 128.41) (end 177.42 127.01) (width 0.25) (layer F.Cu) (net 4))
 (segment (start 185.274 132.4623) (end 183.5223 132.4623) (width 0.25) (layer F.Cu) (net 4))
 (segment (start 182.2396 131.1796) (end 179.686 131.1796) (width 0.25) (layer F.Cu) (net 4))
 (segment (start 183.5223 132.4623) (end 182.2396 131.1796) (width 0.25) (layer F.Cu) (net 4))
 (segment (start 181.53 134.94) (end 181.53 132.7101) (width 0.25) (layer F.Cu) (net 5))
 (segment (start 181.53 132.7101) (end 180.6345 131.8146) (width 0.25) (layer F.Cu) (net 5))
 (segment (start 180.6345 131.8146) (end 179.686 131.8146) (width 0.25) (layer F.Cu) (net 5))
 (segment (start 179.686 131.8146) (end 178.3746 131.8146) (width 0.25) (layer F.Cu) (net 5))
 (segment (start 178.3746 131.8146) (end 177.42 130.86) (width 0.25) (layer F.Cu) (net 5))
 (segment (start 178.167344 124.250708) (end 176.82 124.79) (width 0.5) (layer F.Cu) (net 2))
 (segment (start 176.82 124.79) (end 174.82 125.58) (width 0.5) (layer F.Cu) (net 2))
 (segment (start 174.82 125.58) (end 175.06 125.58) (width 0.25) (layer F.Cu) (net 2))
 (segment (start 174.82 125.58) (end 174.82 128.1) (width 0.25) (layer F.Cu) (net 2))
 (segment (start 174.82 128.1) (end 174.91 128.19) (width 0.25) (layer F.Cu) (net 2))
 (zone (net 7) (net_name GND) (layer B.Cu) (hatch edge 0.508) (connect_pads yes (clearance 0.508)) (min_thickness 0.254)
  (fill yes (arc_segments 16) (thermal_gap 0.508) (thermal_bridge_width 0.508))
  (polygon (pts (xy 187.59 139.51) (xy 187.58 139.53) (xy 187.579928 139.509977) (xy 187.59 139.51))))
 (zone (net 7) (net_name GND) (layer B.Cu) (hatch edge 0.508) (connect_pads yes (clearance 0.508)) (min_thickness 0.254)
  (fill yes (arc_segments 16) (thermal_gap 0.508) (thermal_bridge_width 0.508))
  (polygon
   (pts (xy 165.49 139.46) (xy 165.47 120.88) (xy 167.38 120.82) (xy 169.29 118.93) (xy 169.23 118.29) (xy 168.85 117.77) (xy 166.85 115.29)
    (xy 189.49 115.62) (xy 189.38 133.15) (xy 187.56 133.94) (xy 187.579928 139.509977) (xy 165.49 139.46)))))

